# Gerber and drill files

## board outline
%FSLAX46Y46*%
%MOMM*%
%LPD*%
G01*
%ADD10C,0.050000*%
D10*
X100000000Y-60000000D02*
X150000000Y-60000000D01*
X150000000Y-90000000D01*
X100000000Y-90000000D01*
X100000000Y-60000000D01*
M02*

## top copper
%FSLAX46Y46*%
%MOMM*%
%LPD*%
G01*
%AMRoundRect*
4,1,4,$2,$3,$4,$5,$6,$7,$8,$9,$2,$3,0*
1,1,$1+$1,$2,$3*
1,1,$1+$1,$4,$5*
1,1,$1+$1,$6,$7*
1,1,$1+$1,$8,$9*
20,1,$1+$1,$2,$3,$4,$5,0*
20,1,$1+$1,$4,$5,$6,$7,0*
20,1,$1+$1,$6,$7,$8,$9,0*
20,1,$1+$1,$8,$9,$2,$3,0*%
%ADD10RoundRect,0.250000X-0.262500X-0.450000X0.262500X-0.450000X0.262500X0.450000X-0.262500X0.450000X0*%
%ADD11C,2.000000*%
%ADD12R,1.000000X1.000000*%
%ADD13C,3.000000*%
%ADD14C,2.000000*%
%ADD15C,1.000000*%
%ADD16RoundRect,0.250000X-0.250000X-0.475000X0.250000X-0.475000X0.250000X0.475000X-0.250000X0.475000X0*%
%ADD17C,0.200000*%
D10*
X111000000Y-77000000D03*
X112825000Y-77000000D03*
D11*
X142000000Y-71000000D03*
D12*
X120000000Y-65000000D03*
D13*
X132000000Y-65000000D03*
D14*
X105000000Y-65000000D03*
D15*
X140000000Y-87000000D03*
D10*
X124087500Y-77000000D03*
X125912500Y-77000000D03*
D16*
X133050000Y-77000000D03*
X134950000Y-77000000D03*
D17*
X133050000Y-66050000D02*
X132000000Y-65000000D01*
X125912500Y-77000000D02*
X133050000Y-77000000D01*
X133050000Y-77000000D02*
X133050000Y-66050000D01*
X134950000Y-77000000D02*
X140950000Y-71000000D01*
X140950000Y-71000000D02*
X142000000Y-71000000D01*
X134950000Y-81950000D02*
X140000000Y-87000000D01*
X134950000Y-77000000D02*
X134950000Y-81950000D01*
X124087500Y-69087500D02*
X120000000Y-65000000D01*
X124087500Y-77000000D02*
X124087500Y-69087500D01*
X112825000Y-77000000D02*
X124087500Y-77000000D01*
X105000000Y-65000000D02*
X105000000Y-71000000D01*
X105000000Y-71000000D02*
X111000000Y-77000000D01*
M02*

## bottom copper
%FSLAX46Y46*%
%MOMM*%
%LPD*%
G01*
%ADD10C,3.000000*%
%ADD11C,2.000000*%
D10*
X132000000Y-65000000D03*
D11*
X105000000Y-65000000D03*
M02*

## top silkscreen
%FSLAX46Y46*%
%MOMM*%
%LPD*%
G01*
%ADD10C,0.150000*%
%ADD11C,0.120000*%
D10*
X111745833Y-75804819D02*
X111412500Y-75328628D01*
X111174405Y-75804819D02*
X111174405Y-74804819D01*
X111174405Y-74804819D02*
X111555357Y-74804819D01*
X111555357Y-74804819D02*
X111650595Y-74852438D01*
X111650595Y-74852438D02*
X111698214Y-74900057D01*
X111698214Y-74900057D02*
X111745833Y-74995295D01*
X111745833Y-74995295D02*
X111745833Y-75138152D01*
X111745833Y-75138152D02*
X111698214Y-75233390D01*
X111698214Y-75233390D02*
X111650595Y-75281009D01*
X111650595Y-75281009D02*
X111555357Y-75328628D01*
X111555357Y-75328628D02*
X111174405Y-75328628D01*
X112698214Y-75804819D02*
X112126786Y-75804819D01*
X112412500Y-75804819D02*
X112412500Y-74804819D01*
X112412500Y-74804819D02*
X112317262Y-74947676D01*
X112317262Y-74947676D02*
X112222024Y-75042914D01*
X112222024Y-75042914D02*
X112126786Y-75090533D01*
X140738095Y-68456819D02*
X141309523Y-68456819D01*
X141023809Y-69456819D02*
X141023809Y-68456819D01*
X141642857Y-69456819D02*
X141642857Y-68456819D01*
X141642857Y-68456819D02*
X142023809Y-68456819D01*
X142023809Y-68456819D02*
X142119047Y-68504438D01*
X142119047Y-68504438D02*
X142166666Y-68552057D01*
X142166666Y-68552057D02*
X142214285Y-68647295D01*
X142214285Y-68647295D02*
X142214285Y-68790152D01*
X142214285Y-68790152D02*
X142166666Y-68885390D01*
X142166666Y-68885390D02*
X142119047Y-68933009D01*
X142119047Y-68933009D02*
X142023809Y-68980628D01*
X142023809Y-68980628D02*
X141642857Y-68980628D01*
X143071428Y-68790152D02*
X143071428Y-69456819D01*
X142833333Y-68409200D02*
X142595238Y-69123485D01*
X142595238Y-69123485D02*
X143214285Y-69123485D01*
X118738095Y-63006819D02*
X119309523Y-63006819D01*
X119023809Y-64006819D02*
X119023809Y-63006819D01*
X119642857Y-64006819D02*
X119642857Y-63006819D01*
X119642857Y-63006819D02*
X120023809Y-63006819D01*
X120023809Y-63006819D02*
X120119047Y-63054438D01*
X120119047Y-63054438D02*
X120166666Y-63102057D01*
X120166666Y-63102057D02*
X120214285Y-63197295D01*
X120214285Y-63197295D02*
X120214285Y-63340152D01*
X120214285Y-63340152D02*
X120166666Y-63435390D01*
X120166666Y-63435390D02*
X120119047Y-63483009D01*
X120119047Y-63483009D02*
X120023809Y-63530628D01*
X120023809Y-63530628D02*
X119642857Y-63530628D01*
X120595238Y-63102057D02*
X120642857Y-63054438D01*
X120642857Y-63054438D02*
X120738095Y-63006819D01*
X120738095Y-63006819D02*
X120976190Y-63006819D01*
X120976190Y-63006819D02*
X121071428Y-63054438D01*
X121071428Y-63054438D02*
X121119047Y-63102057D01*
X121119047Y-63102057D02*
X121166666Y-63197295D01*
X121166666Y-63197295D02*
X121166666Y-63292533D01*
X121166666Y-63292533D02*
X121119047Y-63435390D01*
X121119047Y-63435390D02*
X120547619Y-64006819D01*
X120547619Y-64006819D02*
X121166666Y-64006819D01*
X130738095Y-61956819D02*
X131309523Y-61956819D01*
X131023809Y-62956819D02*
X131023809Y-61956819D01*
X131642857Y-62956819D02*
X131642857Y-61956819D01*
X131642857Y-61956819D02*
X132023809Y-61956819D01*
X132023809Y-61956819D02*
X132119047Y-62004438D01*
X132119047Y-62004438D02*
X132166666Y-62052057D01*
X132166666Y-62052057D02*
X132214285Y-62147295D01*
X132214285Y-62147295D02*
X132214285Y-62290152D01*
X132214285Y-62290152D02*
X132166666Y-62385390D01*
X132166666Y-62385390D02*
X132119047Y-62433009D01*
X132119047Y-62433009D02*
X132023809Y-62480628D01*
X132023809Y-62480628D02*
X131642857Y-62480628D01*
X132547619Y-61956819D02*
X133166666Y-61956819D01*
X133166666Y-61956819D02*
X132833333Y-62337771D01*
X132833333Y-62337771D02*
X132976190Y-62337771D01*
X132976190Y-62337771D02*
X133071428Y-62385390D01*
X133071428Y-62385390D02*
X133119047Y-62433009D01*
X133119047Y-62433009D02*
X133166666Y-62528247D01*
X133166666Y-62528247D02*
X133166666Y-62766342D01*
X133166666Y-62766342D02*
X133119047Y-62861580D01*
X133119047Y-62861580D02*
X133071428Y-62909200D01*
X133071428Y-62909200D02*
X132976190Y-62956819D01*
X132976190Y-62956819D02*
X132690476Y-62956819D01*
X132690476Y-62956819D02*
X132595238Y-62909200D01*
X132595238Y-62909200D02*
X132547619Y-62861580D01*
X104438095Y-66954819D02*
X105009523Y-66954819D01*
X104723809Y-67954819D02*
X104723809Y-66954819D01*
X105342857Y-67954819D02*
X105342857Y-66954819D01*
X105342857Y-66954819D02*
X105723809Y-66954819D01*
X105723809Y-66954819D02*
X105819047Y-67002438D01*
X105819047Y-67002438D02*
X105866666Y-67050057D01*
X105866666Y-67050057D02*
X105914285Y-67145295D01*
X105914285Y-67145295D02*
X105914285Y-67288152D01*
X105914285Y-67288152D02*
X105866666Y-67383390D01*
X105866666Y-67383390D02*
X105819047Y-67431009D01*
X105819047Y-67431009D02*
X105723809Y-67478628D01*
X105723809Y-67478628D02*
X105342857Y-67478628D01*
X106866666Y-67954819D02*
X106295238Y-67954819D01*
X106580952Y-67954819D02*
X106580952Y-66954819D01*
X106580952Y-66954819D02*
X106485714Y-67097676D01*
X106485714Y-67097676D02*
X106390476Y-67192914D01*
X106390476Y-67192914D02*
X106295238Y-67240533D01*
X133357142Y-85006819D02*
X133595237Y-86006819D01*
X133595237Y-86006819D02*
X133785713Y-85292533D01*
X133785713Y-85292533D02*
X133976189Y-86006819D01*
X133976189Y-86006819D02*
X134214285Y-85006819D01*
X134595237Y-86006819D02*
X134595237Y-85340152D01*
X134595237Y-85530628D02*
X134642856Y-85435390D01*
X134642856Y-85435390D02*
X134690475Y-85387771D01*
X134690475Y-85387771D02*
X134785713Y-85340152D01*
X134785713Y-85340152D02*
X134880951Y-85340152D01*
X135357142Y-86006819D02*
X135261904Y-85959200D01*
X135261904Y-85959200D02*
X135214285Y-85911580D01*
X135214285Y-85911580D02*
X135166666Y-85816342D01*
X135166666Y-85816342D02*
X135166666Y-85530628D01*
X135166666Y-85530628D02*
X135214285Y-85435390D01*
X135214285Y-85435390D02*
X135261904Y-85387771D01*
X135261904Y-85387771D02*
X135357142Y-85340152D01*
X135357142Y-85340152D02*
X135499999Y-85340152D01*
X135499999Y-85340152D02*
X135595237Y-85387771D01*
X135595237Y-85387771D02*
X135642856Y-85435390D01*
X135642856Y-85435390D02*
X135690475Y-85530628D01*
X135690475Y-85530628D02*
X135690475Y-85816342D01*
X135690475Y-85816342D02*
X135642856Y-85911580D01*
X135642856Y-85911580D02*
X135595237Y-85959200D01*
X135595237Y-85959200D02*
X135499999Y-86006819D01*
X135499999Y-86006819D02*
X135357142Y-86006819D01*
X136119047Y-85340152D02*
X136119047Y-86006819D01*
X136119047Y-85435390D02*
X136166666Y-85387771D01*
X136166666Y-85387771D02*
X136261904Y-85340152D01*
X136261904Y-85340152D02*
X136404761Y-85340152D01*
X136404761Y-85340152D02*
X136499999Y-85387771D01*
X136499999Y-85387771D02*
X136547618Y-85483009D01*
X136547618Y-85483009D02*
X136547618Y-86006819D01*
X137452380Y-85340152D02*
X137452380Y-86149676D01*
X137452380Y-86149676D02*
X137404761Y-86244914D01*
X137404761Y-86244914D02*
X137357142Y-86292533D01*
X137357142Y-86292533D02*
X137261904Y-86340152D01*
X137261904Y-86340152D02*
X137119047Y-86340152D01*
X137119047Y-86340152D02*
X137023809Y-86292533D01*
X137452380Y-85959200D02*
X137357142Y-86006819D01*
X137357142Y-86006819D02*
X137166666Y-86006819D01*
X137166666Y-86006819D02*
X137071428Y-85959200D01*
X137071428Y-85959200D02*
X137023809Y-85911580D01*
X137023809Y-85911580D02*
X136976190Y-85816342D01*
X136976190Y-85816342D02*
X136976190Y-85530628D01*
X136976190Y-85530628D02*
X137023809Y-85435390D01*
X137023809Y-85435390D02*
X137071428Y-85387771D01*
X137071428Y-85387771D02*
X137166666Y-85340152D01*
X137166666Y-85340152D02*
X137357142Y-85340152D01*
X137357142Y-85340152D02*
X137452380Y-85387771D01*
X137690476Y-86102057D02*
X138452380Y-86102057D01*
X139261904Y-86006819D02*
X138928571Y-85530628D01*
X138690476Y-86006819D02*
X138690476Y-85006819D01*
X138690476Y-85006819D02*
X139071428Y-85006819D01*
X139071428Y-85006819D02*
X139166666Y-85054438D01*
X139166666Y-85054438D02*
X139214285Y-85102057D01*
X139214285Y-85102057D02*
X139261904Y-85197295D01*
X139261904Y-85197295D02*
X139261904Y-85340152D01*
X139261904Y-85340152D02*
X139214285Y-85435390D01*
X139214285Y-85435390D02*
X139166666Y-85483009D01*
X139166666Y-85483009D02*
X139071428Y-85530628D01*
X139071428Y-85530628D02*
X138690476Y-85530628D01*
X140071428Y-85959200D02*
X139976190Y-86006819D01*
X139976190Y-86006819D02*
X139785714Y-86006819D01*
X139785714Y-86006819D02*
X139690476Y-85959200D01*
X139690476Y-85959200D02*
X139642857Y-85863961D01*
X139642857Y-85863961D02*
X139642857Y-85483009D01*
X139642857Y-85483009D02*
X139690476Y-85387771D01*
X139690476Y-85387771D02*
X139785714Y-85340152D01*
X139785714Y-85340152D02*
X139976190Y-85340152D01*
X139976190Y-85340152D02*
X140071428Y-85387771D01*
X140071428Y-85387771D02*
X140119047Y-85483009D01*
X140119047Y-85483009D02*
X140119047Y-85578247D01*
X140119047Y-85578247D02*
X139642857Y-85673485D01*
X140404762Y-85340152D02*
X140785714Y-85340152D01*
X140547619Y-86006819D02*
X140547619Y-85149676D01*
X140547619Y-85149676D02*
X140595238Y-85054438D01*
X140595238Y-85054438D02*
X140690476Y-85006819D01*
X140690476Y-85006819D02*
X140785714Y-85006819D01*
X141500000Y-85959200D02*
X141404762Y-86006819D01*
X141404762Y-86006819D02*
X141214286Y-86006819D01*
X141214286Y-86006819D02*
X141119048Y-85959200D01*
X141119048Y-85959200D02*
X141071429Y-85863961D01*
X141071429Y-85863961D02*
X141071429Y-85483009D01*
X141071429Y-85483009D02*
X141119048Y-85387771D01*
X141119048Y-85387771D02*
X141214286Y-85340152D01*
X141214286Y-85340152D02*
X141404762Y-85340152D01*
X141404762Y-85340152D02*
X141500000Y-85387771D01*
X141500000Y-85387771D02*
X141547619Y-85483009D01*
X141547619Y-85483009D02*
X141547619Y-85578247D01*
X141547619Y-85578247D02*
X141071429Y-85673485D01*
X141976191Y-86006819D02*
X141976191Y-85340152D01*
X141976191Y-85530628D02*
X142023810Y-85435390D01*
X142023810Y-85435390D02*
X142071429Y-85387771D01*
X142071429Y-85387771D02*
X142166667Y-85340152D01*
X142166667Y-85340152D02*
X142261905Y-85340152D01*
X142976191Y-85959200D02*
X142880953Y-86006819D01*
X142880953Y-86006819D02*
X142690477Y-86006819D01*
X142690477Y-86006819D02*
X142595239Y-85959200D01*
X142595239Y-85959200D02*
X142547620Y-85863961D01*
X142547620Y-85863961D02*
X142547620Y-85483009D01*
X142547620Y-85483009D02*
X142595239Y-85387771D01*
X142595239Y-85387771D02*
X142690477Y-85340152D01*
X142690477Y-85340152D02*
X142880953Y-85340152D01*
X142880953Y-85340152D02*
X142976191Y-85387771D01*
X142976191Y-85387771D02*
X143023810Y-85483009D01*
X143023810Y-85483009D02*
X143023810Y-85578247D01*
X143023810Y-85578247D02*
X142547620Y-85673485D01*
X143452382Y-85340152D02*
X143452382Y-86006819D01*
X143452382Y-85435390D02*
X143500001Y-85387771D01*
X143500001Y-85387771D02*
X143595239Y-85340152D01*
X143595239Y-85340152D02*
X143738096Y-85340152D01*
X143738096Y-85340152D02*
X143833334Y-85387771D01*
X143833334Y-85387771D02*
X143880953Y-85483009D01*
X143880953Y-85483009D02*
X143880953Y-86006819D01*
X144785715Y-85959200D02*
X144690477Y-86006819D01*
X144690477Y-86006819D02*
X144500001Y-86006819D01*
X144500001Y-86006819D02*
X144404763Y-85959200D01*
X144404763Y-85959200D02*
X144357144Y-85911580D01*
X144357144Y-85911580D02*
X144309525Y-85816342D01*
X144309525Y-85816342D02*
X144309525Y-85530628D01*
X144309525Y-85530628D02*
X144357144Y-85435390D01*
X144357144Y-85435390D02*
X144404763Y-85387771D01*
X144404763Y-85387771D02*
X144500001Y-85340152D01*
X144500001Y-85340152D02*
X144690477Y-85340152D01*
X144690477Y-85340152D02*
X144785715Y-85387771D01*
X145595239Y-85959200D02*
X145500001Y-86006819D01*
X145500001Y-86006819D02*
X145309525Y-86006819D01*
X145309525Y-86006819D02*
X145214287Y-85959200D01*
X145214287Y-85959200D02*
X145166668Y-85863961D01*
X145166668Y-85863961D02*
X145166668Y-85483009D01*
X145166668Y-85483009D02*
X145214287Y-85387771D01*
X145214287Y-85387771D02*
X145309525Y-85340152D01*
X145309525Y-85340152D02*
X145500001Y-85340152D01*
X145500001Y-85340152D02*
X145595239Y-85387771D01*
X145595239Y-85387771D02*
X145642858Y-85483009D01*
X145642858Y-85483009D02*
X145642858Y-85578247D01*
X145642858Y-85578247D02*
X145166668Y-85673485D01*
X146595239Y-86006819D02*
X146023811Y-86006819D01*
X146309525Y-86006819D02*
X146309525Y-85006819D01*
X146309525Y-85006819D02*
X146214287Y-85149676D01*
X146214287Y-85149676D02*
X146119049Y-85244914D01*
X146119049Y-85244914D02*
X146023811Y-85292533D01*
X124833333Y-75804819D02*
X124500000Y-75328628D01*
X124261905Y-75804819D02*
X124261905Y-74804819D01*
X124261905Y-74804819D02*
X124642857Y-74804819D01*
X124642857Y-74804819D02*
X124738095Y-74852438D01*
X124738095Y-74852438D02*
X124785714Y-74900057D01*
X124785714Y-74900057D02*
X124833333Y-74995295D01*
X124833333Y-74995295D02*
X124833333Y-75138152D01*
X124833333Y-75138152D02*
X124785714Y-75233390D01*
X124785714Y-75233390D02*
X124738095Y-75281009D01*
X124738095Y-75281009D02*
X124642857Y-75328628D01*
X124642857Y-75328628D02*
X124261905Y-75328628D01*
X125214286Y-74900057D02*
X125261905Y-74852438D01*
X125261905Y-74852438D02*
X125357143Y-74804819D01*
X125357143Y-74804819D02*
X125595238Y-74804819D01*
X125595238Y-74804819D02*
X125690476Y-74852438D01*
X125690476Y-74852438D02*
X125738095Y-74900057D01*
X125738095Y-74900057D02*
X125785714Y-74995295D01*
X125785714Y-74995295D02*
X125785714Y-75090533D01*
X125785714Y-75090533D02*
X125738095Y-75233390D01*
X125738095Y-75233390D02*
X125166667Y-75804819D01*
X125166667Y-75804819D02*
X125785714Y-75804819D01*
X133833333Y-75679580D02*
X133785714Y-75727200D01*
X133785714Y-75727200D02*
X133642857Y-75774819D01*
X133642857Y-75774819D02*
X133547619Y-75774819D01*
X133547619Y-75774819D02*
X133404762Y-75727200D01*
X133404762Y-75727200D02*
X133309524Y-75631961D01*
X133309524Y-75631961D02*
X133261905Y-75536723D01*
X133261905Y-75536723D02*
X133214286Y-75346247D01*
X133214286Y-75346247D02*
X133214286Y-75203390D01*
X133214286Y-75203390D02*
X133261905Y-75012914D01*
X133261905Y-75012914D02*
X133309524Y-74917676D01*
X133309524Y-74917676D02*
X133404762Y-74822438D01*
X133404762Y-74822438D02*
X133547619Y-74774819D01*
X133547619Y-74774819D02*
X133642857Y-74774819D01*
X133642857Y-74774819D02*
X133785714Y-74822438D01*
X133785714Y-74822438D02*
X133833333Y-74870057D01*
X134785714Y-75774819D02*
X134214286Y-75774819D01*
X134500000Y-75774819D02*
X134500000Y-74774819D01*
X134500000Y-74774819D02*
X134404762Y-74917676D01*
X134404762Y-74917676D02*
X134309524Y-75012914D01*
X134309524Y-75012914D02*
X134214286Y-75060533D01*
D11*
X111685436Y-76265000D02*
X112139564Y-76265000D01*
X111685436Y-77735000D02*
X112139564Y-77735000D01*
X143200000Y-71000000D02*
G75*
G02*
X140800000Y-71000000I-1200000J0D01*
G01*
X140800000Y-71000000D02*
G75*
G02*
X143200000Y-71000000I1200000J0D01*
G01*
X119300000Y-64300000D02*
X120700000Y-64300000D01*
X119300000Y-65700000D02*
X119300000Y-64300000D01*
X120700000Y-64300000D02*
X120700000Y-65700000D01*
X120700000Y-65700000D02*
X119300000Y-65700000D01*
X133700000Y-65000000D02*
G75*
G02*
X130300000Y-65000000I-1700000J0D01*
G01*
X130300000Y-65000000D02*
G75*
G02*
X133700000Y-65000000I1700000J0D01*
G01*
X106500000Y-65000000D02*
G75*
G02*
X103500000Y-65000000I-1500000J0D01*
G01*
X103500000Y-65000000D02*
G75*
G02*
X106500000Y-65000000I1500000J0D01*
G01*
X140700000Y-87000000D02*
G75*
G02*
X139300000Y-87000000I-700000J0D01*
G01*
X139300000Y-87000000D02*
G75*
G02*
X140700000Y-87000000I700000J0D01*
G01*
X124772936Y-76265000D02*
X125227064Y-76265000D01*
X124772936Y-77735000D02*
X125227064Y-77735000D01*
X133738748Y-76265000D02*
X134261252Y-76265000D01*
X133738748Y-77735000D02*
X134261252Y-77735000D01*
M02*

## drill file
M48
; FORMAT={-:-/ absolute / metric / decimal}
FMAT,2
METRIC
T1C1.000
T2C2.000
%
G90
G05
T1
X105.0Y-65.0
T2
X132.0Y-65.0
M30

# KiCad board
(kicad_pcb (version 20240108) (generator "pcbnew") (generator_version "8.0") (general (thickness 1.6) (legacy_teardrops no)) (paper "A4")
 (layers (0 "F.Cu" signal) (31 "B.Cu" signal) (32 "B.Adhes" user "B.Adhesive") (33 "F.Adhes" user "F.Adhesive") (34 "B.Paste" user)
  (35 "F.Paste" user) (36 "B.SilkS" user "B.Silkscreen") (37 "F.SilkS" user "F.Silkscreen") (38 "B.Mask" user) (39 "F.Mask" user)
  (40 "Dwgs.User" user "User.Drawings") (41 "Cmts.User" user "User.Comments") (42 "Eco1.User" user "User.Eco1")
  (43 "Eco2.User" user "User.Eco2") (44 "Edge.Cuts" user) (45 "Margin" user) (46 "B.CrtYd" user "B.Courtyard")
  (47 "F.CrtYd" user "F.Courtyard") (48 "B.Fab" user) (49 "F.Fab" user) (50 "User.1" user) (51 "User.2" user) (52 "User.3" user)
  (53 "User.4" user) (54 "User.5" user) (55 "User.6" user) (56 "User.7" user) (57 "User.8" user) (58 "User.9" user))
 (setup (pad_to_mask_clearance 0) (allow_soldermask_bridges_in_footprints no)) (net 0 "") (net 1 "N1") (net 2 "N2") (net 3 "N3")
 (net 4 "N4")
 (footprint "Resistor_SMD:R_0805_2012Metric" (layer "F.Cu") (at 111.9125 77)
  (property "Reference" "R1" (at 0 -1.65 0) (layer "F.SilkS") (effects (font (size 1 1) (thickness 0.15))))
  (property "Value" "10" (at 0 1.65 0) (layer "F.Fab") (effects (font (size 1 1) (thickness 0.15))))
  (fp_line (start -0.227064 -0.735) (end 0.227064 -0.735) (stroke (width 0.12) (type solid)) (layer "F.SilkS"))
  (fp_line (start -0.227064 0.735) (end 0.227064 0.735) (stroke (width 0.12) (type solid)) (layer "F.SilkS"))
  (pad "1" smd roundrect (at -0.9125 0) (size 1.025 1.4) (layers "F.Cu" "F.Paste" "F.Mask") (roundrect_rratio 0.243902) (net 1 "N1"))
  (pad "2" smd roundrect (at 0.9125 0) (size 1.025 1.4) (layers "F.Cu" "F.Paste" "F.Mask") (roundrect_rratio 0.243902) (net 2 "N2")))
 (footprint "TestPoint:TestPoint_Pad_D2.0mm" (layer "F.Cu") (at 142 71)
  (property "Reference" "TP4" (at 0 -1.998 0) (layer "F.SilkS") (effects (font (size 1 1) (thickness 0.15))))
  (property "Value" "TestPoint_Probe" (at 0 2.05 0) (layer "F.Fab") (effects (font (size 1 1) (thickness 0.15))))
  (fp_circle (center 0 0) (end 0 1.2) (stroke (width 0.12) (type solid)) (fill none) (layer "F.SilkS"))
  (pad "1" smd circle (at 0 0) (size 2 2) (layers "F.Cu" "F.Mask") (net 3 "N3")))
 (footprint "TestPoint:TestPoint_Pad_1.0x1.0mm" (layer "F.Cu") (at 120 65)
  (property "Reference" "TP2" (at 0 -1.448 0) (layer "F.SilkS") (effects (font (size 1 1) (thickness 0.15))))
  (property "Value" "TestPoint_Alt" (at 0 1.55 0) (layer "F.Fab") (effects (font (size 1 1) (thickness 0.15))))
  (fp_line (start -0.7 -0.7) (end 0.7 -0.7) (stroke (width 0.12) (type solid)) (layer "F.SilkS"))
  (fp_line (start -0.7 0.7) (end -0.7 -0.7) (stroke (width 0.12) (type solid)) (layer "F.SilkS"))
  (fp_line (start 0.7 -0.7) (end 0.7 0.7) (stroke (width 0.12) (type solid)) (layer "F.SilkS"))
  (fp_line (start 0.7 0.7) (end -0.7 0.7) (stroke (width 0.12) (type solid)) (layer "F.SilkS"))
  (pad "1" smd rect (at 0 0) (size 1 1) (layers "F.Cu" "F.Mask") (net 2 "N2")))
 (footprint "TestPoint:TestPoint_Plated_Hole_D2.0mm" (layer "F.Cu") (at 132 65)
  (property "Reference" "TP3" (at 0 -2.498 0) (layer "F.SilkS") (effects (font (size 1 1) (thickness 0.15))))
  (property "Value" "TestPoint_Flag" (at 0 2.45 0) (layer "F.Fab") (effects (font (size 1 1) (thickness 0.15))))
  (fp_circle (center 0 0) (end 0 -1.7) (stroke (width 0.12) (type solid)) (fill none) (layer "F.SilkS"))
  (pad "1" thru_hole circle (at 0 0) (size 3 3) (drill 2) (layers "*.Cu" "*.Mask") (remove_unused_layers no) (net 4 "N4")))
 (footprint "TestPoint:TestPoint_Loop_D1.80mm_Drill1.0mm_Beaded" (layer "F.Cu") (at 105 65)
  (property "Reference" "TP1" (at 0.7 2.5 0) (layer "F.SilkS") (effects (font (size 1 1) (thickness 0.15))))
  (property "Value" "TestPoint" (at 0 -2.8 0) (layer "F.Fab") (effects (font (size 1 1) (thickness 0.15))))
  (fp_circle (center 0 0) (end 1.5 0) (stroke (width 0.12) (type solid)) (fill none) (layer "F.SilkS"))
  (pad "1" thru_hole circle (at 0 0) (size 2 2) (drill 1) (layers "*.Cu" "*.Mask") (remove_unused_layers no) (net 1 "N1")))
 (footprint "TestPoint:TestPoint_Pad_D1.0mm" (layer "F.Cu") (at 140 87)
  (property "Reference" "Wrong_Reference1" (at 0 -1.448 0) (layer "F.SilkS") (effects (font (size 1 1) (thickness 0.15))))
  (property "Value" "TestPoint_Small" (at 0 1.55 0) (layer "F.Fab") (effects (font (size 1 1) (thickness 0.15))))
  (fp_circle (center 0 0) (end 0 0.7) (stroke (width 0.12) (type solid)) (fill none) (layer "F.SilkS"))
  (pad "1" smd circle (at 0 0) (size 1 1) (layers "F.Cu" "F.Mask") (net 3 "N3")))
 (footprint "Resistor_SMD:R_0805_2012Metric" (layer "F.Cu") (at 125 77)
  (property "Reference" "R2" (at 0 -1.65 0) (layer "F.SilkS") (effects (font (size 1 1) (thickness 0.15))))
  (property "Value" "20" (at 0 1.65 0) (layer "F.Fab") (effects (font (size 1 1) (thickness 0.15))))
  (fp_line (start -0.227064 -0.735) (end 0.227064 -0.735) (stroke (width 0.12) (type solid)) (layer "F.SilkS"))
  (fp_line (start -0.227064 0.735) (end 0.227064 0.735) (stroke (width 0.12) (type solid)) (layer "F.SilkS"))
  (pad "1" smd roundrect (at -0.9125 0) (size 1.025 1.4) (layers "F.Cu" "F.Paste" "F.Mask") (roundrect_rratio 0.243902) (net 2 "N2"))
  (pad "2" smd roundrect (at 0.9125 0) (size 1.025 1.4) (layers "F.Cu" "F.Paste" "F.Mask") (roundrect_rratio 0.243902) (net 4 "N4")))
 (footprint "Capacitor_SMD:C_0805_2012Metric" (layer "F.Cu") (at 134 77)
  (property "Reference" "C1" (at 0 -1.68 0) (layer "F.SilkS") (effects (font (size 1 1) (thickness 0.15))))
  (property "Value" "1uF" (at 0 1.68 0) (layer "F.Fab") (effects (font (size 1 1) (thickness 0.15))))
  (fp_line (start -0.261252 -0.735) (end 0.261252 -0.735) (stroke (width 0.12) (type solid)) (layer "F.SilkS"))
  (fp_line (start -0.261252 0.735) (end 0.261252 0.735) (stroke (width 0.12) (type solid)) (layer "F.SilkS"))
  (pad "1" smd roundrect (at -0.95 0) (size 1 1.45) (layers "F.Cu" "F.Paste" "F.Mask") (roundrect_rratio 0.25) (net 4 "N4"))
  (pad "2" smd roundrect (at 0.95 0) (size 1 1.45) (layers "F.Cu" "F.Paste" "F.Mask") (roundrect_rratio 0.25) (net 3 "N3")))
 (gr_rect (start 100 60) (end 150 90) (stroke (width 0.05) (type default)) (fill none) (layer "Edge.Cuts"))
 (segment (start 133.05 66.05) (end 132 65) (width 0.2) (layer "F.Cu") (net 4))
 (segment (start 125.9125 77) (end 133.05 77) (width 0.2) (layer "F.Cu") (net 4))
 (segment (start 133.05 77) (end 133.05 66.05) (width 0.2) (layer "F.Cu") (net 4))
 (segment (start 134.95 77) (end 140.95 71) (width 0.2) (layer "F.Cu") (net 3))
 (segment (start 140.95 71) (end 142 71) (width 0.2) (layer "F.Cu") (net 3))
 (segment (start 134.95 81.95) (end 140 87) (width 0.2) (layer "F.Cu") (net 3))
 (segment (start 134.95 77) (end 134.95 81.95) (width 0.2) (layer "F.Cu") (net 3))
 (segment (start 124.0875 69.0875) (end 120 65) (width 0.2) (layer "F.Cu") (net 2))
 (segment (start 124.0875 77) (end 124.0875 69.0875) (width 0.2) (layer "F.Cu") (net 2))
 (segment (start 112.825 77) (end 124.0875 77) (width 0.2) (layer "F.Cu") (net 2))
 (segment (start 105 65) (end 105 71) (width 0.2) (layer "F.Cu") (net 1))
 (segment (start 105 71) (end 111 77) (width 0.2) (layer "F.Cu") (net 1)))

